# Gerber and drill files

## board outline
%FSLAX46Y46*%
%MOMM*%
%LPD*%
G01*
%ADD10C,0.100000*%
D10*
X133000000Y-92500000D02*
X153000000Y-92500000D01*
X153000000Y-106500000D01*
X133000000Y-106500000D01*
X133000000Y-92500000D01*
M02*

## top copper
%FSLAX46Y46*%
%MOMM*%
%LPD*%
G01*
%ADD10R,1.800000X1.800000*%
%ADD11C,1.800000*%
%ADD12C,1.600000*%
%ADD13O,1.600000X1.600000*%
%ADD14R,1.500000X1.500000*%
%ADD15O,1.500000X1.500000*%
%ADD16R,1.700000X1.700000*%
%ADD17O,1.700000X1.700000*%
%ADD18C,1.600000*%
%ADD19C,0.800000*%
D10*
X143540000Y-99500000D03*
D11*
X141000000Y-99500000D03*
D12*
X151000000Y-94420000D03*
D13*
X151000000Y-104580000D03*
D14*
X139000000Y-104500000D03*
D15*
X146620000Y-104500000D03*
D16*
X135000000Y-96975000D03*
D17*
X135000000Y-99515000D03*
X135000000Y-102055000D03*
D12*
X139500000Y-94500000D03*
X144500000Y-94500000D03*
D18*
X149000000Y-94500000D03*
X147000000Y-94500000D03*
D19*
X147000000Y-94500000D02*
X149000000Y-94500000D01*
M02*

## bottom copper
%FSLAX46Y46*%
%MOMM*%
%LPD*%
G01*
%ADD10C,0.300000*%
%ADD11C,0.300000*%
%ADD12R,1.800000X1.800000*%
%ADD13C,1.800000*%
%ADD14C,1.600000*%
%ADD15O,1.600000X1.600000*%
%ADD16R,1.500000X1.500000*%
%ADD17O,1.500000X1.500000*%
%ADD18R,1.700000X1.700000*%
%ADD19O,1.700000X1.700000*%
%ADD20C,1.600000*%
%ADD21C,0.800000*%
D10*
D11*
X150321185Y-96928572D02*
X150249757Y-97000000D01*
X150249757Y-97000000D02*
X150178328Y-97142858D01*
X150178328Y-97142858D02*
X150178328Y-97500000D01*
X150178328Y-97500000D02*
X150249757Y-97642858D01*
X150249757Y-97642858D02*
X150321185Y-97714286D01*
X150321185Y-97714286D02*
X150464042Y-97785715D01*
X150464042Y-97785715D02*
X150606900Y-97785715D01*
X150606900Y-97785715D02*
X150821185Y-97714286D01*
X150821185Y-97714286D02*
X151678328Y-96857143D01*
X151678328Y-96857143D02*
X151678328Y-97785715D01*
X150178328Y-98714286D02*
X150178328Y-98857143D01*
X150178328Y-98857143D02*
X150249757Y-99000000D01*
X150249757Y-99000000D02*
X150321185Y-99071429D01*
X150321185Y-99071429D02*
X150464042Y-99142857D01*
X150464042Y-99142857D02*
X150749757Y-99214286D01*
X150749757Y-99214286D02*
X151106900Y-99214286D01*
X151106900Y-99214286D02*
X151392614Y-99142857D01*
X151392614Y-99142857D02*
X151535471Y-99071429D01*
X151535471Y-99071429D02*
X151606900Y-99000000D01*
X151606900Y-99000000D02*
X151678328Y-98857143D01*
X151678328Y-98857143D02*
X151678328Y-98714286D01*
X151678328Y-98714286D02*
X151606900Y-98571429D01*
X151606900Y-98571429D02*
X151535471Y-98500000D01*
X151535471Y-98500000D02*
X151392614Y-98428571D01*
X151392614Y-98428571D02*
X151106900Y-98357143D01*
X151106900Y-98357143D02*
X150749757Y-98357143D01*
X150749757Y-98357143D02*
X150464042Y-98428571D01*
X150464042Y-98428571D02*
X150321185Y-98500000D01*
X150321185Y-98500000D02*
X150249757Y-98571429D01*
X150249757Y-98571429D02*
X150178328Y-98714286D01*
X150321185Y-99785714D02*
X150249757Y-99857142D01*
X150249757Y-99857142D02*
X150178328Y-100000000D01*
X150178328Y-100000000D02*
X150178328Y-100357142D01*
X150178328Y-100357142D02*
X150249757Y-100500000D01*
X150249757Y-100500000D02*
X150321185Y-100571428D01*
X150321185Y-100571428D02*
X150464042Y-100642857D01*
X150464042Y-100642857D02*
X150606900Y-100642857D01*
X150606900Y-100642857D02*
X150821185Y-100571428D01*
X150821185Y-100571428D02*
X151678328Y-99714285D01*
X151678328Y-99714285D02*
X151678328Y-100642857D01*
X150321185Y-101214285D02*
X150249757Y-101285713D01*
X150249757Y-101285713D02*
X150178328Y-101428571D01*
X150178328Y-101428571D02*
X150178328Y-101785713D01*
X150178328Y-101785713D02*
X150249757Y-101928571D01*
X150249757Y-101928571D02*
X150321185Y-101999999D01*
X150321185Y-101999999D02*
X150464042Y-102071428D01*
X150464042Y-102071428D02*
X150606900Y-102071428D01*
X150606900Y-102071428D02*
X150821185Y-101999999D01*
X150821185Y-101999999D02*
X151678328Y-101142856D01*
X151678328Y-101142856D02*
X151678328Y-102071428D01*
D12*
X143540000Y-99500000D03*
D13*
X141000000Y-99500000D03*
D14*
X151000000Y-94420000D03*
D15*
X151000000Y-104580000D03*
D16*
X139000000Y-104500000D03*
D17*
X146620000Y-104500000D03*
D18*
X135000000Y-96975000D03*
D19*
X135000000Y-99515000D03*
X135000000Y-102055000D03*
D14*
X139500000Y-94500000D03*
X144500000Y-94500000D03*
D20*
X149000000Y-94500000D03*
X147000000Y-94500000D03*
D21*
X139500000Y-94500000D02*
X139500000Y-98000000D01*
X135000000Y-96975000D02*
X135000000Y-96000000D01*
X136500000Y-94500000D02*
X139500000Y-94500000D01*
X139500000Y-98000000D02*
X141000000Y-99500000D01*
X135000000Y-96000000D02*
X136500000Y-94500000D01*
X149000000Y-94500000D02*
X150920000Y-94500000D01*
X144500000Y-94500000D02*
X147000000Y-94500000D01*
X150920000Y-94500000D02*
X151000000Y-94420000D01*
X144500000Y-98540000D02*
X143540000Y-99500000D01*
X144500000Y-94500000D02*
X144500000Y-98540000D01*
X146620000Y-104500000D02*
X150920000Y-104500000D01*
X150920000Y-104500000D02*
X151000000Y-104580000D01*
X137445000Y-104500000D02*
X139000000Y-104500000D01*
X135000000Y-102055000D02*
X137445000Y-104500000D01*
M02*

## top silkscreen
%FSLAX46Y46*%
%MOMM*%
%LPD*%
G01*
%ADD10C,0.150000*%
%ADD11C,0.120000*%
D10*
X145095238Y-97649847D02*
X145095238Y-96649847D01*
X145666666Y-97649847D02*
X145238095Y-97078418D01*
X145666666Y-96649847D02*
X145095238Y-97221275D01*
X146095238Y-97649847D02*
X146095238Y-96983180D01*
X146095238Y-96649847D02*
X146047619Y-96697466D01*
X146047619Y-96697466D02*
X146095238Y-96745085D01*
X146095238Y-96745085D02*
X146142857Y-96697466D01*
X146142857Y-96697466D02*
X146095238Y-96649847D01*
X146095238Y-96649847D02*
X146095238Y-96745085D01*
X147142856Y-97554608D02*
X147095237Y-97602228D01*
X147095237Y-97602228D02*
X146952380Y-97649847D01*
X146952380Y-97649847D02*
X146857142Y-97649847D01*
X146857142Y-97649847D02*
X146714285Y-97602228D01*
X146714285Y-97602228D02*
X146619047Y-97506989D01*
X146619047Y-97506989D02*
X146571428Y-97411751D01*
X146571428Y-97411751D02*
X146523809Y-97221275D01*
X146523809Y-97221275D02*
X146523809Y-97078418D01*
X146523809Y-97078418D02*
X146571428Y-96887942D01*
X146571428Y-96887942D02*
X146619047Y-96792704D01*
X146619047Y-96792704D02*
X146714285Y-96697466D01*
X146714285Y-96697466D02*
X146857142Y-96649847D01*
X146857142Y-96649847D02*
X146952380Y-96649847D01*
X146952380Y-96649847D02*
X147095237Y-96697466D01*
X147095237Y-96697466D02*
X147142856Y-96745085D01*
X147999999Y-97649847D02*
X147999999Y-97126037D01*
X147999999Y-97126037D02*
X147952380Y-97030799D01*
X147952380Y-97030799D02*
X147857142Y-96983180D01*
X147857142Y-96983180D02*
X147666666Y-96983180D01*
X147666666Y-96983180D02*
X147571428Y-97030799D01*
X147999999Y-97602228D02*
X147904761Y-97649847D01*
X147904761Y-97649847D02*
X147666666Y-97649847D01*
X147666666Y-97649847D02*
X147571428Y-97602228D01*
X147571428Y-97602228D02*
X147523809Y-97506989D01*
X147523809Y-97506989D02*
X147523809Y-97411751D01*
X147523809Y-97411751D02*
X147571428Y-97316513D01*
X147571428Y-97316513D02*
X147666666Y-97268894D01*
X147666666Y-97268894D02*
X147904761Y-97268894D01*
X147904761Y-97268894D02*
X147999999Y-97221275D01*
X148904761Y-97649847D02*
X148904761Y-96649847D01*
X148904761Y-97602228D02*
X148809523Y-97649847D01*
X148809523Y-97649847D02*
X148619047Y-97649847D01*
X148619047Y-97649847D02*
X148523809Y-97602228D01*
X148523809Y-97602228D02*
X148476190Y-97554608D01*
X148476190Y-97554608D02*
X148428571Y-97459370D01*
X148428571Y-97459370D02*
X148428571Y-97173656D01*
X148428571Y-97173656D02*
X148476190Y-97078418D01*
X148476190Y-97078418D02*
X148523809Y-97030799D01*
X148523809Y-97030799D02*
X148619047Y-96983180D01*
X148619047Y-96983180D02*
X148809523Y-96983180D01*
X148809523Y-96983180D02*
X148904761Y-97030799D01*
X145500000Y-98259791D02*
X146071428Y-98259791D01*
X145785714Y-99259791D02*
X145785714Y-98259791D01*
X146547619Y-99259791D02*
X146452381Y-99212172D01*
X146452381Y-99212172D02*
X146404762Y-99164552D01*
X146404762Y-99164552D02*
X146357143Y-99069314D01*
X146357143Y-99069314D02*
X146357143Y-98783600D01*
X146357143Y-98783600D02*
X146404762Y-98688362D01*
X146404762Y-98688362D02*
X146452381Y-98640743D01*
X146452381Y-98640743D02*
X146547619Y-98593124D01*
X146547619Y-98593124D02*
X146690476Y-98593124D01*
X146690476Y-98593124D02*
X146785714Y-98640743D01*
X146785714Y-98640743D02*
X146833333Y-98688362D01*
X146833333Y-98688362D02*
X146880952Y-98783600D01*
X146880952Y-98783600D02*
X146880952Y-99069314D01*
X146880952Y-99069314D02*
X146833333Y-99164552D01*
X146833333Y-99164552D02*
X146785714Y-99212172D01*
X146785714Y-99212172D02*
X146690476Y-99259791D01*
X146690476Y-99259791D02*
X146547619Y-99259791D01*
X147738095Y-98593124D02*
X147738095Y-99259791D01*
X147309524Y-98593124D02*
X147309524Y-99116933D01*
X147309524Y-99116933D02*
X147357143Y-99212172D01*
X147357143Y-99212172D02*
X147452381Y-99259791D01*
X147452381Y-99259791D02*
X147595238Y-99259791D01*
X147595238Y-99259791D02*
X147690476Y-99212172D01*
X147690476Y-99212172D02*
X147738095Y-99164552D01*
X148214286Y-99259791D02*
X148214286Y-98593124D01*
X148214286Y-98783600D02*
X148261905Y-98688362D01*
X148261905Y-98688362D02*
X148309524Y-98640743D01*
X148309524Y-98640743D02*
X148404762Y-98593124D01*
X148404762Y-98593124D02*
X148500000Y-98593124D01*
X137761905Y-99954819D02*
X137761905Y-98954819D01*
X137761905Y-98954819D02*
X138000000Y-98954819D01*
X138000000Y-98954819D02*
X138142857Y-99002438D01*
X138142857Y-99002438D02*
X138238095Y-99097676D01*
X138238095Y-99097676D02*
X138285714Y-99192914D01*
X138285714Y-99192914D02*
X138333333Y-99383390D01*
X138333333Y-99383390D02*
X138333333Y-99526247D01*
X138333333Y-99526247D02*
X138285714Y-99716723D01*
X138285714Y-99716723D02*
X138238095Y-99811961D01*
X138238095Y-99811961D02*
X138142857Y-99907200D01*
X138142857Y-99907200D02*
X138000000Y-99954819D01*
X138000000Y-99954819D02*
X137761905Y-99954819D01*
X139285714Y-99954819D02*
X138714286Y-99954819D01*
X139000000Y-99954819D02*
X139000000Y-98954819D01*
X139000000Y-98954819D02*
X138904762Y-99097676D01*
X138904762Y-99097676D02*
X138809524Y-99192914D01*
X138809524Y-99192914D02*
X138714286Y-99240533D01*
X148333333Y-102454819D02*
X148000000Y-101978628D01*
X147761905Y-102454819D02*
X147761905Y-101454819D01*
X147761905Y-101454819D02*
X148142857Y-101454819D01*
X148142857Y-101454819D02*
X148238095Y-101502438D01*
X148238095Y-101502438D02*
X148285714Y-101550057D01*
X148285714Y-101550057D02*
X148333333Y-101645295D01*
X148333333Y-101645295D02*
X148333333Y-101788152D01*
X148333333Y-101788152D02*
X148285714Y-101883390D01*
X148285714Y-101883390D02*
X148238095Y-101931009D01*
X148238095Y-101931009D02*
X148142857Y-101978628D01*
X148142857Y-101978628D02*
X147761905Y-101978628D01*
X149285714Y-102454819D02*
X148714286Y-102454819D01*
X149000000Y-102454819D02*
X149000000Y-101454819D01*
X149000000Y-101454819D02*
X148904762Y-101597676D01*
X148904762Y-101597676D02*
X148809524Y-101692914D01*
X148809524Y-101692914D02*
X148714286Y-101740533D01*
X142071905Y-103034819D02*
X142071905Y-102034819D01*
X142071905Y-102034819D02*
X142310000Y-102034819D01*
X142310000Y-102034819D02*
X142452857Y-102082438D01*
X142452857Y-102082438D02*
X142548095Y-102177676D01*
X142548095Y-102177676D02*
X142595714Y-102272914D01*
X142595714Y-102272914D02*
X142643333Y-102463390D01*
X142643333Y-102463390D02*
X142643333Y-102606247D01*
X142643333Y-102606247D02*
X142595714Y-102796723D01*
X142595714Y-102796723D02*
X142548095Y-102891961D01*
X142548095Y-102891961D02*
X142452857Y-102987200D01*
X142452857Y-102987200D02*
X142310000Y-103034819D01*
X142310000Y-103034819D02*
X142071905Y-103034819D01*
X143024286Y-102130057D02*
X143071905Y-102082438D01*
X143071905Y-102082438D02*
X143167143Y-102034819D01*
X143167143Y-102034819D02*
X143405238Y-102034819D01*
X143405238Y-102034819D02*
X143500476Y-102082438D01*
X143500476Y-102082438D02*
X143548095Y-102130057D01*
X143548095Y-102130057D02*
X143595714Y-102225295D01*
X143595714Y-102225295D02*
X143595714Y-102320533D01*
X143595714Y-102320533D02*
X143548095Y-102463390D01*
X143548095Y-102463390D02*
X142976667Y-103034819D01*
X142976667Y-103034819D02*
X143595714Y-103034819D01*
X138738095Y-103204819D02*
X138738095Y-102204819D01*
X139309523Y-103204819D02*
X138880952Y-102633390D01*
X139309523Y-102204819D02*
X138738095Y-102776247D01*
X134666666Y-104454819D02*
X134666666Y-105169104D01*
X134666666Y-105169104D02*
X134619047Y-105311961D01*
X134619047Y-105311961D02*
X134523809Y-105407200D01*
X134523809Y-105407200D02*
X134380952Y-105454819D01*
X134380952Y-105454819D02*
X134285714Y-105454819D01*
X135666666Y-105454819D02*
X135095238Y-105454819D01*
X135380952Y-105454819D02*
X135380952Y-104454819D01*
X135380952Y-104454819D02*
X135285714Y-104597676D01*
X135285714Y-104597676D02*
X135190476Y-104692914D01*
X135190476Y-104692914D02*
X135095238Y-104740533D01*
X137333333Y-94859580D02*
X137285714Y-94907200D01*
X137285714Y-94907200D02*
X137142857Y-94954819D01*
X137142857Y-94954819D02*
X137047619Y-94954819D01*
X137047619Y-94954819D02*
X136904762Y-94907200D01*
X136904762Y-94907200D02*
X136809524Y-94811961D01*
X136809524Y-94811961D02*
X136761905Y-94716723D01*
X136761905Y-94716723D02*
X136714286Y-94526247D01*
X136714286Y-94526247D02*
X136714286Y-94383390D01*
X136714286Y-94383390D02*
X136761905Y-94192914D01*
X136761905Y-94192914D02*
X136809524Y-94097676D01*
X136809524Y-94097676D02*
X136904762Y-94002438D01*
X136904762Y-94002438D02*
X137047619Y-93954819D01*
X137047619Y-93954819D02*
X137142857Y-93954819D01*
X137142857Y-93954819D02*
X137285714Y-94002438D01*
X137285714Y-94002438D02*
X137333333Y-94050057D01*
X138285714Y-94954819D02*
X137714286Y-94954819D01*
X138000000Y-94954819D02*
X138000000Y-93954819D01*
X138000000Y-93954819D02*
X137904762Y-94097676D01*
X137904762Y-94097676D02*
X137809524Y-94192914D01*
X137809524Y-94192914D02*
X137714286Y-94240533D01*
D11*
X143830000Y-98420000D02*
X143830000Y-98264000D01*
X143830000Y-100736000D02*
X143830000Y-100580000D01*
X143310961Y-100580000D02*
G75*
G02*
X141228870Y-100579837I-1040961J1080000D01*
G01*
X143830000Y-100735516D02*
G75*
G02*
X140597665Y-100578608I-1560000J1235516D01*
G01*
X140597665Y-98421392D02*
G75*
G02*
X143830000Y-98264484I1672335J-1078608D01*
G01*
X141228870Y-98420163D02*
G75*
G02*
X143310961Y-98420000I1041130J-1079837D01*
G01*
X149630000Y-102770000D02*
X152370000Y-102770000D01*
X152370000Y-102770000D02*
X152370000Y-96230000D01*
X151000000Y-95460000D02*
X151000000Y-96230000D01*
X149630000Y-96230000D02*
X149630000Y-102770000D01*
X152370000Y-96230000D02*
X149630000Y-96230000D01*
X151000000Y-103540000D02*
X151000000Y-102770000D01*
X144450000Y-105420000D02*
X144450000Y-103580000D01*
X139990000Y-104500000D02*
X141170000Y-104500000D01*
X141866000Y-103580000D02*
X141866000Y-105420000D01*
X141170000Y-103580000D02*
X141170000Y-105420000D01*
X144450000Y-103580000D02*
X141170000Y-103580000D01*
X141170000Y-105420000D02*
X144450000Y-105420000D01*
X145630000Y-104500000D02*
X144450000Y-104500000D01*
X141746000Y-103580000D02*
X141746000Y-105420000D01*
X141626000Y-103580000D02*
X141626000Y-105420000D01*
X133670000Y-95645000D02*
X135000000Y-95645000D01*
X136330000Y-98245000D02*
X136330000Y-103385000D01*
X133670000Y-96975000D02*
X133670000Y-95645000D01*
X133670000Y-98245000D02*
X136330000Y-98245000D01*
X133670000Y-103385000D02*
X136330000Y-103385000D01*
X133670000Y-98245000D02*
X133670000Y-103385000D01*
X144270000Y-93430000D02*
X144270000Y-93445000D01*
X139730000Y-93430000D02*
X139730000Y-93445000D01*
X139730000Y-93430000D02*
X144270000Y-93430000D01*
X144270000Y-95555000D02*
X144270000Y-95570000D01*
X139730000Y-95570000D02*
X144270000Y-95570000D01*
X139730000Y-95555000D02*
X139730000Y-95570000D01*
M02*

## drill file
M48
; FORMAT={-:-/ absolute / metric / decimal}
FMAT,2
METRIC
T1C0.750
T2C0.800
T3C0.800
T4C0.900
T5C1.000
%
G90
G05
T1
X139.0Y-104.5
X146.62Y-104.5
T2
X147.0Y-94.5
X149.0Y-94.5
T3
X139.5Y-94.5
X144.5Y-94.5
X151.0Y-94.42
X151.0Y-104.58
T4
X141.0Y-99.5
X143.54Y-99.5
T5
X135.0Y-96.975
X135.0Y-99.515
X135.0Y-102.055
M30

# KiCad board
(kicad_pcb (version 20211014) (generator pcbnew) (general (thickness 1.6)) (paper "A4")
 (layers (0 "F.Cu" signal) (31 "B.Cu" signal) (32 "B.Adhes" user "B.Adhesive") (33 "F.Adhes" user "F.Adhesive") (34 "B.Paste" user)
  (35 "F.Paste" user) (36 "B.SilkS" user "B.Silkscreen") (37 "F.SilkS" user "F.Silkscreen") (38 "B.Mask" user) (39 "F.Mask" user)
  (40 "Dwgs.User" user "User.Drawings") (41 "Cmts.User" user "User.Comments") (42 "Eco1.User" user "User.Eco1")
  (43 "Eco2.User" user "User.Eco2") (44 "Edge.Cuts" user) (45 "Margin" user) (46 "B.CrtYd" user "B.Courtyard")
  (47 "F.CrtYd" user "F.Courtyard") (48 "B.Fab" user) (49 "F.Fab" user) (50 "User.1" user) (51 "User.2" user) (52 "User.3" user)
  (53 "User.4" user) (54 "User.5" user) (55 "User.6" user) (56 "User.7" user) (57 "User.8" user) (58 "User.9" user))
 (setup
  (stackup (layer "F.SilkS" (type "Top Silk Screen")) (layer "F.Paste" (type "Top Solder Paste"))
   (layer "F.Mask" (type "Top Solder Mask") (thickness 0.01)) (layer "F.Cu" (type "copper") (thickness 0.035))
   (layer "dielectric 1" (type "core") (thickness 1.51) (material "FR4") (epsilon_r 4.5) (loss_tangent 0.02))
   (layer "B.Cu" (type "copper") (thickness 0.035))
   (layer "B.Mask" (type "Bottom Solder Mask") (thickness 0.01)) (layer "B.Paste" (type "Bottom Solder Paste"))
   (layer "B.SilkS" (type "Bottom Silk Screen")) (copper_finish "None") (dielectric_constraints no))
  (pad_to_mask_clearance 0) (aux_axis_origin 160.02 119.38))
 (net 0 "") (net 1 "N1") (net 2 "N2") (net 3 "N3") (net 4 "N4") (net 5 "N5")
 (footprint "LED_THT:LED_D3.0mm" (layer "F.Cu") (at 143.54 99.5 180)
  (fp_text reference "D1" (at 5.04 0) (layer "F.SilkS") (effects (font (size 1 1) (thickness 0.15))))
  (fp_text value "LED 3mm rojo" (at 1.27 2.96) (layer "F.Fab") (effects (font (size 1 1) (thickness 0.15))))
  (fp_line (start -0.29 1.08) (end -0.29 1.236) (layer "F.SilkS") (width 0.12))
  (fp_line (start -0.29 -1.236) (end -0.29 -1.08) (layer "F.SilkS") (width 0.12))
  (fp_arc (start 0.229039 -1.08) (mid 1.270117 -1.5) (end 2.31113 -1.079837) (layer "F.SilkS") (width 0.12))
  (fp_arc (start -0.29 -1.235516) (mid 1.366487 -1.987659) (end 2.942335 -1.078608) (layer "F.SilkS") (width 0.12))
  (fp_arc (start 2.942335 1.078608) (mid 1.366487 1.987659) (end -0.29 1.235516) (layer "F.SilkS") (width 0.12))
  (fp_arc (start 2.31113 1.079837) (mid 1.270117 1.5) (end 0.229039 1.08) (layer "F.SilkS") (width 0.12))
  (pad "1" thru_hole rect (at 0 0 180) (size 1.8 1.8) (drill 0.9) (layers *.Cu *.Mask) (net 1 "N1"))
  (pad "2" thru_hole circle (at 2.54 0 180) (size 1.8 1.8) (drill 0.9) (layers *.Cu *.Mask) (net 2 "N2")))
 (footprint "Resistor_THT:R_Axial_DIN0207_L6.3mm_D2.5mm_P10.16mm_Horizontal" (layer "F.Cu") (at 151 94.42 -90)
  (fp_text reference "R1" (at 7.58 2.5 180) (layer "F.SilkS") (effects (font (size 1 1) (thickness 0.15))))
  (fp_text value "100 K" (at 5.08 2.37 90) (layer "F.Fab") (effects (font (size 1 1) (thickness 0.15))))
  (fp_line (start 8.35 1.37) (end 8.35 -1.37) (layer "F.SilkS") (width 0.12))
  (fp_line (start 8.35 -1.37) (end 1.81 -1.37) (layer "F.SilkS") (width 0.12))
  (fp_line (start 1.04 0) (end 1.81 0) (layer "F.SilkS") (width 0.12))
  (fp_line (start 1.81 1.37) (end 8.35 1.37) (layer "F.SilkS") (width 0.12))
  (fp_line (start 1.81 -1.37) (end 1.81 1.37) (layer "F.SilkS") (width 0.12))
  (fp_line (start 9.12 0) (end 8.35 0) (layer "F.SilkS") (width 0.12))
  (pad "1" thru_hole circle (at 0 0 270) (size 1.6 1.6) (drill 0.8) (layers *.Cu *.Mask) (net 1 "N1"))
  (pad "2" thru_hole oval (at 10.16 0 270) (size 1.6 1.6) (drill 0.8) (layers *.Cu *.Mask) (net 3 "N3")))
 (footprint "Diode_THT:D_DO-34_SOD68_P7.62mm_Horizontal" (layer "F.Cu") (at 139 104.5)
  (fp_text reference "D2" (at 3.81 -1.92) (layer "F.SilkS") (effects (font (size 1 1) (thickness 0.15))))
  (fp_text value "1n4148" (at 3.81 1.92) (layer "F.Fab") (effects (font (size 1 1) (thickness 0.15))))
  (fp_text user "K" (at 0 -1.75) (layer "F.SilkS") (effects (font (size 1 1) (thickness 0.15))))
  (fp_line (start 5.45 0.92) (end 5.45 -0.92) (layer "F.SilkS") (width 0.12))
  (fp_line (start 0.99 0) (end 2.17 0) (layer "F.SilkS") (width 0.12))
  (fp_line (start 2.866 -0.92) (end 2.866 0.92) (layer "F.SilkS") (width 0.12))
  (fp_line (start 2.17 -0.92) (end 2.17 0.92) (layer "F.SilkS") (width 0.12))
  (fp_line (start 5.45 -0.92) (end 2.17 -0.92) (layer "F.SilkS") (width 0.12))
  (fp_line (start 2.17 0.92) (end 5.45 0.92) (layer "F.SilkS") (width 0.12))
  (fp_line (start 6.63 0) (end 5.45 0) (layer "F.SilkS") (width 0.12))
  (fp_line (start 2.746 -0.92) (end 2.746 0.92) (layer "F.SilkS") (width 0.12))
  (fp_line (start 2.626 -0.92) (end 2.626 0.92) (layer "F.SilkS") (width 0.12))
  (pad "1" thru_hole rect (at 0 0) (size 1.5 1.5) (drill 0.75) (layers *.Cu *.Mask) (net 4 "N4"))
  (pad "2" thru_hole oval (at 7.62 0) (size 1.5 1.5) (drill 0.75) (layers *.Cu *.Mask) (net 3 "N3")))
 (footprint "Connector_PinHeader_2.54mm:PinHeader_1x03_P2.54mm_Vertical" (layer "F.Cu") (at 135 96.975)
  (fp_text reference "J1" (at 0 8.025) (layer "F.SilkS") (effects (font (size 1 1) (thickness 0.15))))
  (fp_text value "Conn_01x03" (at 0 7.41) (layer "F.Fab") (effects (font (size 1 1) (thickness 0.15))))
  (fp_line (start -1.33 -1.33) (end 0 -1.33) (layer "F.SilkS") (width 0.12))
  (fp_line (start 1.33 1.27) (end 1.33 6.41) (layer "F.SilkS") (width 0.12))
  (fp_line (start -1.33 0) (end -1.33 -1.33) (layer "F.SilkS") (width 0.12))
  (fp_line (start -1.33 1.27) (end 1.33 1.27) (layer "F.SilkS") (width 0.12))
  (fp_line (start -1.33 6.41) (end 1.33 6.41) (layer "F.SilkS") (width 0.12))
  (fp_line (start -1.33 1.27) (end -1.33 6.41) (layer "F.SilkS") (width 0.12))
  (pad "1" thru_hole rect (at 0 0) (size 1.7 1.7) (drill 1) (layers *.Cu *.Mask) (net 2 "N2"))
  (pad "2" thru_hole oval (at 0 2.54) (size 1.7 1.7) (drill 1) (layers *.Cu *.Mask) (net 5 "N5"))
  (pad "3" thru_hole oval (at 0 5.08) (size 1.7 1.7) (drill 1) (layers *.Cu *.Mask) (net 4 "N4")))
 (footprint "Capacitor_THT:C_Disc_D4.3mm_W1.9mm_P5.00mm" (layer "F.Cu") (at 139.5 94.5)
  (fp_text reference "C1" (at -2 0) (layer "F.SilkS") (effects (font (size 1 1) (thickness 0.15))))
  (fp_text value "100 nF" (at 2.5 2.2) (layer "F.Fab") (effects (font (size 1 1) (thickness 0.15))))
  (fp_line (start 4.77 -1.07) (end 4.77 -1.055) (layer "F.SilkS") (width 0.12))
  (fp_line (start 0.23 -1.07) (end 0.23 -1.055) (layer "F.SilkS") (width 0.12))
  (fp_line (start 0.23 -1.07) (end 4.77 -1.07) (layer "F.SilkS") (width 0.12))
  (fp_line (start 4.77 1.055) (end 4.77 1.07) (layer "F.SilkS") (width 0.12))
  (fp_line (start 0.23 1.07) (end 4.77 1.07) (layer "F.SilkS") (width 0.12))
  (fp_line (start 0.23 1.055) (end 0.23 1.07) (layer "F.SilkS") (width 0.12))
  (pad "1" thru_hole circle (at 0 0) (size 1.6 1.6) (drill 0.8) (layers *.Cu *.Mask) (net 2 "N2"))
  (pad "2" thru_hole circle (at 5 0) (size 1.6 1.6) (drill 0.8) (layers *.Cu *.Mask) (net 1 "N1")))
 (gr_rect (start 133 92.5) (end 153 106.5) (layer "Edge.Cuts") (width 0.1) (fill none))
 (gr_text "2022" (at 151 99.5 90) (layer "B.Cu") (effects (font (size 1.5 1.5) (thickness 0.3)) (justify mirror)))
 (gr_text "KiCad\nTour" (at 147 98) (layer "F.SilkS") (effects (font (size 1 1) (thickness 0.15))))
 (segment (start 139.5 94.5) (end 139.5 98) (width 0.8) (layer "B.Cu") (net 2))
 (segment (start 135 96.975) (end 135 96) (width 0.8) (layer "B.Cu") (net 2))
 (segment (start 136.5 94.5) (end 139.5 94.5) (width 0.8) (layer "B.Cu") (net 2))
 (segment (start 139.5 98) (end 141 99.5) (width 0.8) (layer "B.Cu") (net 2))
 (segment (start 135 96) (end 136.5 94.5) (width 0.8) (layer "B.Cu") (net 2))
 (segment (start 147 94.5) (end 149 94.5) (width 0.8) (layer "F.Cu") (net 1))
 (via (at 149 94.5) (size 1.6) (drill 0.8) (layers "F.Cu" "B.Cu") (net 1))
 (via (at 147 94.5) (size 1.6) (drill 0.8) (layers "F.Cu" "B.Cu") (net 1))
 (segment (start 149 94.5) (end 150.92 94.5) (width 0.8) (layer "B.Cu") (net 1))
 (segment (start 144.5 94.5) (end 147 94.5) (width 0.8) (layer "B.Cu") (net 1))
 (segment (start 150.92 94.5) (end 151 94.42) (width 0.8) (layer "B.Cu") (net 1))
 (segment (start 144.5 98.54) (end 143.54 99.5) (width 0.8) (layer "B.Cu") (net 1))
 (segment (start 144.5 94.5) (end 144.5 98.54) (width 0.8) (layer "B.Cu") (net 1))
 (segment (start 146.62 104.5) (end 150.92 104.5) (width 0.8) (layer "B.Cu") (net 3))
 (segment (start 150.92 104.5) (end 151 104.58) (width 0.8) (layer "B.Cu") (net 3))
 (segment (start 137.445 104.5) (end 139 104.5) (width 0.8) (layer "B.Cu") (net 4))
 (segment (start 135 102.055) (end 137.445 104.5) (width 0.8) (layer "B.Cu") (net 4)))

